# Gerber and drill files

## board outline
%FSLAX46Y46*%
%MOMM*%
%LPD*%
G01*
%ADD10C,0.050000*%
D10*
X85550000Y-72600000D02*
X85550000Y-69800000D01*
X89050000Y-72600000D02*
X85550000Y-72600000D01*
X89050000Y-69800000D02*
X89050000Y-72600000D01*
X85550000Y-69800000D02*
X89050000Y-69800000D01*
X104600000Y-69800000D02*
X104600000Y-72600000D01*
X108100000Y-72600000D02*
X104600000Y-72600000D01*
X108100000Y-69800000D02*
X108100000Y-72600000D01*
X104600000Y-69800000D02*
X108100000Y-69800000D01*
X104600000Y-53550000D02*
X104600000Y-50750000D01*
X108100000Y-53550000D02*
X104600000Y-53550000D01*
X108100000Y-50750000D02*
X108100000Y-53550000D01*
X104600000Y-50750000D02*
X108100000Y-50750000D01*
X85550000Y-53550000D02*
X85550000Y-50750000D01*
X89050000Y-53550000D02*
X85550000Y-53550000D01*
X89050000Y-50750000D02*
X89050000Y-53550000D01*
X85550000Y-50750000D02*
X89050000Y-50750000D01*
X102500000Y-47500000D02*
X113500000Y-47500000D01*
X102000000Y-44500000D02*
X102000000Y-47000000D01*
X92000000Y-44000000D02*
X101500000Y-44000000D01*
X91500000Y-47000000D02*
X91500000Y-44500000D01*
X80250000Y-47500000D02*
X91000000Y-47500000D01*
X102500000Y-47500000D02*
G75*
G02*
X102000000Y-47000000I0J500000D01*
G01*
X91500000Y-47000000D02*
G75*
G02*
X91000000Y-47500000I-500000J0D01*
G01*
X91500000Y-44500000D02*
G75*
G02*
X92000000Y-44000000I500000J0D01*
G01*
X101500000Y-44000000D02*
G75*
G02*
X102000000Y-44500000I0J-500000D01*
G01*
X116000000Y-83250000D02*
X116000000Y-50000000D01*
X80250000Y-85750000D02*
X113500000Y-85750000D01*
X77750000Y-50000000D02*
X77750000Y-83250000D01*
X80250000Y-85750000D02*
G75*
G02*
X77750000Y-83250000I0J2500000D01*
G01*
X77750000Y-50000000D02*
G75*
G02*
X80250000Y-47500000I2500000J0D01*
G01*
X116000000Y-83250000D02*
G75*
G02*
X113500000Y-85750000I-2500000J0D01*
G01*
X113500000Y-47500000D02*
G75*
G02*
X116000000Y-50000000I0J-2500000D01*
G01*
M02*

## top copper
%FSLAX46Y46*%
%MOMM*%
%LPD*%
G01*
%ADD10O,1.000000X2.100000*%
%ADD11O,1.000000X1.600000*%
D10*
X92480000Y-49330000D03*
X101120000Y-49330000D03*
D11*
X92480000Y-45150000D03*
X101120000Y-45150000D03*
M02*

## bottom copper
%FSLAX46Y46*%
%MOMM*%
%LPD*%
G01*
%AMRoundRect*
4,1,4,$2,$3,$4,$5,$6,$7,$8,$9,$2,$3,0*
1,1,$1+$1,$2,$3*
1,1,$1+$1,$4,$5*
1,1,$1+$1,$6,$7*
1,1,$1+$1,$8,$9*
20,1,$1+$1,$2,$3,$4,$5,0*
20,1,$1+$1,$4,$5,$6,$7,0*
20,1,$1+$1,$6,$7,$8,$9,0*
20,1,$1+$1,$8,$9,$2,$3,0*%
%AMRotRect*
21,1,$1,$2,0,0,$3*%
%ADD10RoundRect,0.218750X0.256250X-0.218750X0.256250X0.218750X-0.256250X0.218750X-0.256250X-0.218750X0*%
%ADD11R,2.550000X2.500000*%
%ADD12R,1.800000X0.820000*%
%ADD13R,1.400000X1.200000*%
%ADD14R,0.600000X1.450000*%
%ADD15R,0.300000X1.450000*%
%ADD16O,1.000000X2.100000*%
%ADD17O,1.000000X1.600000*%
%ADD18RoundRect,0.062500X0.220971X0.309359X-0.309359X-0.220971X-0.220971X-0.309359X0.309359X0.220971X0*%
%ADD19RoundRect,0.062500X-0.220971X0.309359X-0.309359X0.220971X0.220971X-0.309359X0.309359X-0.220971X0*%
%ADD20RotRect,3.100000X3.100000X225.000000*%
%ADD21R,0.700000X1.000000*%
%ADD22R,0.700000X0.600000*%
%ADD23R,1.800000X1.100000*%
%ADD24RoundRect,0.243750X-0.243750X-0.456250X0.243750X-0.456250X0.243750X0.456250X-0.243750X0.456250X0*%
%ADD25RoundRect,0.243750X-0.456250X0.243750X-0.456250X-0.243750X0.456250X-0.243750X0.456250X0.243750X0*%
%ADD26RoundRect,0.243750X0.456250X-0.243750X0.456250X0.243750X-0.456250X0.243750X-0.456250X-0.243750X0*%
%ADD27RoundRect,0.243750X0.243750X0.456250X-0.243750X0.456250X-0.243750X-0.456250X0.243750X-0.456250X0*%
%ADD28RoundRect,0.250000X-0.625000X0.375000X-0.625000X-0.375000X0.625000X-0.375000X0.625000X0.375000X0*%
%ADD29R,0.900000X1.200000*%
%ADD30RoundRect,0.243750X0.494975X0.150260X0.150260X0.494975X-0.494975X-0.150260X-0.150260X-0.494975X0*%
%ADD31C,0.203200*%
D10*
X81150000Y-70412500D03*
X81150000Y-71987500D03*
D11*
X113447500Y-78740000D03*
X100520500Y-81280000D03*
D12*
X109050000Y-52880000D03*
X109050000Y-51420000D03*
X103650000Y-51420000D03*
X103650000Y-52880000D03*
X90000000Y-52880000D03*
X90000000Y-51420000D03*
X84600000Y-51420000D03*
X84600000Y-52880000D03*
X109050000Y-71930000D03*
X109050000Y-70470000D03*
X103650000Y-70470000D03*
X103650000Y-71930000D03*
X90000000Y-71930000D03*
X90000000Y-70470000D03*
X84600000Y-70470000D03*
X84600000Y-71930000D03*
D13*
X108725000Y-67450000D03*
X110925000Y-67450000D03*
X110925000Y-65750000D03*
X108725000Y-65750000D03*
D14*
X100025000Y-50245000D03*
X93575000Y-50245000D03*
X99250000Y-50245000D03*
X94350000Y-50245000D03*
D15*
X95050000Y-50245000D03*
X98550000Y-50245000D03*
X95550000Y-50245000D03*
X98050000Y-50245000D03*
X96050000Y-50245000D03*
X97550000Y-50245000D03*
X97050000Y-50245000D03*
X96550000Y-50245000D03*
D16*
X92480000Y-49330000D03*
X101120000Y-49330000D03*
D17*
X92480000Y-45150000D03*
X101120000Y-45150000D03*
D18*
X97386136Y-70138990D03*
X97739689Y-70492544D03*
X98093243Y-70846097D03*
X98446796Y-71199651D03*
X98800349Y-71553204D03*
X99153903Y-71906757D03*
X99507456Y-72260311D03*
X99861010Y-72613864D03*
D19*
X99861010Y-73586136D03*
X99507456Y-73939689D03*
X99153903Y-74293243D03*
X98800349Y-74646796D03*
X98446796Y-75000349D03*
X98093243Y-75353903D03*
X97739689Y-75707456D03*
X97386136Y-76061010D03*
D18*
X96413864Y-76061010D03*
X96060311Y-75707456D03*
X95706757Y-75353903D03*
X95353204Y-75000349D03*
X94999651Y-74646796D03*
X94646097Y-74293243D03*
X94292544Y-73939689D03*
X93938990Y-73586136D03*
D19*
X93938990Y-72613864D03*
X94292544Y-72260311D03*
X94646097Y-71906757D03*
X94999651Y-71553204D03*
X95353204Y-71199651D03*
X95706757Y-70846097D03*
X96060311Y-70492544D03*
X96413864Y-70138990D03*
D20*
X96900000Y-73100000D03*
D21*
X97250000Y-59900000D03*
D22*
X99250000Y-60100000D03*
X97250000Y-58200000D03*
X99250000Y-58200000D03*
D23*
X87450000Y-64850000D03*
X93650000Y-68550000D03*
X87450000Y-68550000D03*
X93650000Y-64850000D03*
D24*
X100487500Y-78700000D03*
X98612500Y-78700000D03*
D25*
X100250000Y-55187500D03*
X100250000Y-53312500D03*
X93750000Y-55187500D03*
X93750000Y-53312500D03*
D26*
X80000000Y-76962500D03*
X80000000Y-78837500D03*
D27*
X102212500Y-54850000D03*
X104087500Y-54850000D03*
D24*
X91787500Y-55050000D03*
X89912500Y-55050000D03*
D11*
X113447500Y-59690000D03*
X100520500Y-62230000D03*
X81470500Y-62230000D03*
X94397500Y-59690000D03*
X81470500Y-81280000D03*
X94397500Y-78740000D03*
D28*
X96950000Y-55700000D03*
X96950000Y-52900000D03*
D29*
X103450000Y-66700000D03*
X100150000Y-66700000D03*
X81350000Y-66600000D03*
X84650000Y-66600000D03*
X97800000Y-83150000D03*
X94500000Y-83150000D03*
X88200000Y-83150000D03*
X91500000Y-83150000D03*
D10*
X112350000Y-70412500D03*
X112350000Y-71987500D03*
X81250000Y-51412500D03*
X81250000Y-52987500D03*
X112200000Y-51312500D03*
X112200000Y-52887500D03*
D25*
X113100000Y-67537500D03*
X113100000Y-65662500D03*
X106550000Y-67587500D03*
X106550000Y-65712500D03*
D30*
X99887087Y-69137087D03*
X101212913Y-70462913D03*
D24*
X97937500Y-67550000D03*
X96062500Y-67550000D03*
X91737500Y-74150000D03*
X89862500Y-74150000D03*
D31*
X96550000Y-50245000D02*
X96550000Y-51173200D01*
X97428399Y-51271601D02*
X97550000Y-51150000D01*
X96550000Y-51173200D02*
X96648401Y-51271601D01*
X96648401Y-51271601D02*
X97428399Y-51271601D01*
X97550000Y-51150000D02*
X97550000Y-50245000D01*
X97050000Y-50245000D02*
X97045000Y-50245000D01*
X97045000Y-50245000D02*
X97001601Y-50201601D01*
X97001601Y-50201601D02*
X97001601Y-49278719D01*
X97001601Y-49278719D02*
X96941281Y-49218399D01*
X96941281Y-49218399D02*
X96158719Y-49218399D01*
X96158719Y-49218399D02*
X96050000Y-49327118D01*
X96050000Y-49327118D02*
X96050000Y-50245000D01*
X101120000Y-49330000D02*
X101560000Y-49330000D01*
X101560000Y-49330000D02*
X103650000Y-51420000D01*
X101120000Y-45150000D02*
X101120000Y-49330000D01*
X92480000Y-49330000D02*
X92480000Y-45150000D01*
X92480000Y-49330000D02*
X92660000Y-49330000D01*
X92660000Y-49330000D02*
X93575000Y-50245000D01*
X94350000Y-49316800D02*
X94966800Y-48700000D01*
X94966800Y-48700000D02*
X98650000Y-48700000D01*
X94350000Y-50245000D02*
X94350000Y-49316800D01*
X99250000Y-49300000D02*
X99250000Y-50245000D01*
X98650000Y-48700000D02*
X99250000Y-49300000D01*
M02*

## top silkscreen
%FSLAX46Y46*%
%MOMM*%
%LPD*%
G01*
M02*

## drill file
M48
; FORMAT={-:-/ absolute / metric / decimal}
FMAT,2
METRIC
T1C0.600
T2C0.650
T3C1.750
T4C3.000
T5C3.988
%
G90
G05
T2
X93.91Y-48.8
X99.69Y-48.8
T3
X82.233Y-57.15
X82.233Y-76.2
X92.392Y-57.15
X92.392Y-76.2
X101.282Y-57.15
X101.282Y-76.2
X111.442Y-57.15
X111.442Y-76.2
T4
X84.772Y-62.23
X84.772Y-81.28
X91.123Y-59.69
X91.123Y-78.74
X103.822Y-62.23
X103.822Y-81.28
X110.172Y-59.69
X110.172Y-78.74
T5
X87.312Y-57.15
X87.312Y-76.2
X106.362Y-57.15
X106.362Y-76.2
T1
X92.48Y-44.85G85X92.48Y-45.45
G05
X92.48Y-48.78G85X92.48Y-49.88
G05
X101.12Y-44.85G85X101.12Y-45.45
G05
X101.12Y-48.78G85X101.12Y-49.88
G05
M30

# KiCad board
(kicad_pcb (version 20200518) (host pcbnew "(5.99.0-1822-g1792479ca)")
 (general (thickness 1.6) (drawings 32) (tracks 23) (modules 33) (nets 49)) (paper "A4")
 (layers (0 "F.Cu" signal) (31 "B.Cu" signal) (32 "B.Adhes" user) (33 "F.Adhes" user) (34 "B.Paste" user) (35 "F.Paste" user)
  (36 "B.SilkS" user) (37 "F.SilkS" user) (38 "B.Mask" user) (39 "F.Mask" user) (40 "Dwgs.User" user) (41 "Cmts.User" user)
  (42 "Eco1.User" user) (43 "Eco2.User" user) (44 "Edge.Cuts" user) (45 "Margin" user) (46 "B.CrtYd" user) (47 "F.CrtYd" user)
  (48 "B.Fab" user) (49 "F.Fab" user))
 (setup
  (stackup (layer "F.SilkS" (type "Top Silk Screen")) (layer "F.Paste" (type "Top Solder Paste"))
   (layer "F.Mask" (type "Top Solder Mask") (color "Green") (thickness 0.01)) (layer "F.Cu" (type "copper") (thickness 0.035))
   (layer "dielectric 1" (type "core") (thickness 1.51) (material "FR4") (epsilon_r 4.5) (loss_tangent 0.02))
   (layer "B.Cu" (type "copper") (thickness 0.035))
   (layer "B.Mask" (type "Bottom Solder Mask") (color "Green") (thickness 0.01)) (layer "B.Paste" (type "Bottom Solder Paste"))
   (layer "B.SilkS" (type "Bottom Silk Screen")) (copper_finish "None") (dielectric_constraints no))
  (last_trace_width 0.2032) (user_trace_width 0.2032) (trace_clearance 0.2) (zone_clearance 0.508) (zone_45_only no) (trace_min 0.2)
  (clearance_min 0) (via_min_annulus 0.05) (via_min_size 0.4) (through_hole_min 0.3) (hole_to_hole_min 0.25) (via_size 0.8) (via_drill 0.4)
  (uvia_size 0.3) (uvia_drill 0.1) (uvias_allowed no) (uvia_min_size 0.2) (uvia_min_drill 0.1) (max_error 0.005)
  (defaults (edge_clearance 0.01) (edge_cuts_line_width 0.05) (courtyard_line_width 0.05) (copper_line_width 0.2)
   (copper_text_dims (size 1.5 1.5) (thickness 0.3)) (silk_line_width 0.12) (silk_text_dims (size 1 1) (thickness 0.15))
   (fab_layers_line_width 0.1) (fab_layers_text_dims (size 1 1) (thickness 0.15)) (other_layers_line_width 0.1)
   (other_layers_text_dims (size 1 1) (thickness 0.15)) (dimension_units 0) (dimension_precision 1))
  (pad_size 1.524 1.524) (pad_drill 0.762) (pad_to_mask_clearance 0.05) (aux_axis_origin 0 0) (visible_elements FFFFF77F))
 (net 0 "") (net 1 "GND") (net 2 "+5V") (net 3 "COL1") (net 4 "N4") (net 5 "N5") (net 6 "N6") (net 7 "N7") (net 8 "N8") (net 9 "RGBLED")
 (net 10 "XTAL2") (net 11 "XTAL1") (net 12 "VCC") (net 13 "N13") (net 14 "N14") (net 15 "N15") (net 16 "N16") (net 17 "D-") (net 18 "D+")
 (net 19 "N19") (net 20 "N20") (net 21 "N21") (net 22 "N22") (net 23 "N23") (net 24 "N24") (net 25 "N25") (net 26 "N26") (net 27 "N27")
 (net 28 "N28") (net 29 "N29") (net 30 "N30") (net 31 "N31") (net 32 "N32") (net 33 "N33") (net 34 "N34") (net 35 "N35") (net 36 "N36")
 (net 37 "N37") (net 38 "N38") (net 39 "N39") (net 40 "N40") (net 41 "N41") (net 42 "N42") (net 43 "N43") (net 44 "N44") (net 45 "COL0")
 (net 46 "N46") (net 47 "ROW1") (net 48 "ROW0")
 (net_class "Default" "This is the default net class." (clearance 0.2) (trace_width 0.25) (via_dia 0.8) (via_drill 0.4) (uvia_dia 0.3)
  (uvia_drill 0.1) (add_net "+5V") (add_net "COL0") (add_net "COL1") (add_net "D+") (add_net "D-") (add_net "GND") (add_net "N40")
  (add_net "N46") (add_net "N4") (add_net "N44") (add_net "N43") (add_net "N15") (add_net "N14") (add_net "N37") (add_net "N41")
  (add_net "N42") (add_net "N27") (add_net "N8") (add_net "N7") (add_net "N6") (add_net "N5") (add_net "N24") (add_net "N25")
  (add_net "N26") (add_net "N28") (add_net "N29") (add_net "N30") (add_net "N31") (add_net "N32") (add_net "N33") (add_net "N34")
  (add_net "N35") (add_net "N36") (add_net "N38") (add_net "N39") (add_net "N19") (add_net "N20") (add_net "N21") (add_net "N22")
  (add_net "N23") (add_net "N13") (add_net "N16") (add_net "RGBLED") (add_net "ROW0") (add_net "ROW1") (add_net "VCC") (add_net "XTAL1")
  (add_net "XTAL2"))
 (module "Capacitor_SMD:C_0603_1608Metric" (layer "B.Cu") (at 81.15 71.2 90)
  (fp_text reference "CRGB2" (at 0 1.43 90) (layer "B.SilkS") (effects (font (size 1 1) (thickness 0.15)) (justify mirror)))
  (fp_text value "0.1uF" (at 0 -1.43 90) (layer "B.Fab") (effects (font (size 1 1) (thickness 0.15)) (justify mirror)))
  (pad "2" smd roundrect (at 0.7875 0 90) (size 0.875 0.95) (layers "B.Cu" "B.Paste" "B.Mask") (roundrect_rratio 0.25) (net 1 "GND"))
  (pad "1" smd roundrect (at -0.7875 0 90) (size 0.875 0.95) (layers "B.Cu" "B.Paste" "B.Mask") (roundrect_rratio 0.25) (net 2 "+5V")))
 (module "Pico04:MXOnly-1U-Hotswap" (layer "F.Cu") (at 106.3625 76.2 180)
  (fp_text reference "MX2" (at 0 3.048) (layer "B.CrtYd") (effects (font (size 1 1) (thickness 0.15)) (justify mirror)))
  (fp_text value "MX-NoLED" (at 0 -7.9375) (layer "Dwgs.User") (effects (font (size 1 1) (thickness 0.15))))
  (pad "" np_thru_hole circle (at 2.54 -5.08 180) (size 3 3) (drill 3) (layers *.Cu *.Mask))
  (pad "" np_thru_hole circle (at 0 0 180) (size 3.9878 3.9878) (drill 3.9878) (layers *.Cu *.Mask))
  (pad "" np_thru_hole circle (at -3.81 -2.54 180) (size 3 3) (drill 3) (layers *.Cu *.Mask))
  (pad "" np_thru_hole circle (at -5.08 0 228.0996) (size 1.75 1.75) (drill 1.75) (layers *.Cu *.Mask))
  (pad "" np_thru_hole circle (at 5.08 0 228.0996) (size 1.75 1.75) (drill 1.75) (layers *.Cu *.Mask))
  (pad "1" smd rect (at -7.085 -2.54 180) (size 2.55 2.5) (layers "B.Cu" "B.Paste" "B.Mask") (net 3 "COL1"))
  (pad "2" smd rect (at 5.842 -5.08 180) (size 2.55 2.5) (layers "B.Cu" "B.Paste" "B.Mask") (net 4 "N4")))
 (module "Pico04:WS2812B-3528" (layer "B.Cu") (at 106.35 52.15)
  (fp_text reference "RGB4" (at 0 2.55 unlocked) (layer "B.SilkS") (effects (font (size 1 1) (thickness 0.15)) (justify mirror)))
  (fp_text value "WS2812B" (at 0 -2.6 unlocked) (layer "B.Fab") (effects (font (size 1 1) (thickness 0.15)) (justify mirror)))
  (pad "1" smd rect (at 2.7 0.73) (size 1.8 0.82) (layers "B.Cu" "B.Paste" "B.Mask") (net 2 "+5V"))
  (pad "2" smd rect (at 2.7 -0.73) (size 1.8 0.82) (layers "B.Cu" "B.Paste" "B.Mask") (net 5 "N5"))
  (pad "3" smd rect (at -2.7 -0.73) (size 1.8 0.82) (layers "B.Cu" "B.Paste" "B.Mask") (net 1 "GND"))
  (pad "4" smd rect (at -2.7 0.73) (size 1.8 0.82) (layers "B.Cu" "B.Paste" "B.Mask") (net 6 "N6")))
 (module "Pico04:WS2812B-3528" (layer "B.Cu") (at 87.3 52.15)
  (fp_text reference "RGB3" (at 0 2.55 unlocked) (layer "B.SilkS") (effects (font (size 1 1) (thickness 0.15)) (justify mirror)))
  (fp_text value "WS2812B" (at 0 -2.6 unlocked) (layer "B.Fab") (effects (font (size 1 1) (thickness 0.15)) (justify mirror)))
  (pad "1" smd rect (at 2.7 0.73) (size 1.8 0.82) (layers "B.Cu" "B.Paste" "B.Mask") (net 2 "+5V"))
  (pad "2" smd rect (at 2.7 -0.73) (size 1.8 0.82) (layers "B.Cu" "B.Paste" "B.Mask") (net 6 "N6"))
  (pad "3" smd rect (at -2.7 -0.73) (size 1.8 0.82) (layers "B.Cu" "B.Paste" "B.Mask") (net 1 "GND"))
  (pad "4" smd rect (at -2.7 0.73) (size 1.8 0.82) (layers "B.Cu" "B.Paste" "B.Mask") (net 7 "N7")))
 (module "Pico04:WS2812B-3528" (layer "B.Cu") (at 106.35 71.2)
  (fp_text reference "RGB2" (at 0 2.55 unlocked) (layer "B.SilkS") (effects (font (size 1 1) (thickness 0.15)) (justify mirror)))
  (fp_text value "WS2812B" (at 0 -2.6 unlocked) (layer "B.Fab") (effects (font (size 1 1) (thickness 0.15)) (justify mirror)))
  (pad "1" smd rect (at 2.7 0.73) (size 1.8 0.82) (layers "B.Cu" "B.Paste" "B.Mask") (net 2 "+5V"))
  (pad "2" smd rect (at 2.7 -0.73) (size 1.8 0.82) (layers "B.Cu" "B.Paste" "B.Mask") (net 7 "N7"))
  (pad "3" smd rect (at -2.7 -0.73) (size 1.8 0.82) (layers "B.Cu" "B.Paste" "B.Mask") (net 1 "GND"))
  (pad "4" smd rect (at -2.7 0.73) (size 1.8 0.82) (layers "B.Cu" "B.Paste" "B.Mask") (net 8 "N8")))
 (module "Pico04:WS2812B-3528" (layer "B.Cu") (at 87.3 71.2)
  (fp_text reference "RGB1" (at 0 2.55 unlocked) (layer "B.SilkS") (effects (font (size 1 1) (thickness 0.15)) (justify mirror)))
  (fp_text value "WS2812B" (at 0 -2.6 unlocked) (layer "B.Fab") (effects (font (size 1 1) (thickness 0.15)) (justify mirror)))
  (pad "1" smd rect (at 2.7 0.73) (size 1.8 0.82) (layers "B.Cu" "B.Paste" "B.Mask") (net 2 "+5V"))
  (pad "2" smd rect (at 2.7 -0.73) (size 1.8 0.82) (layers "B.Cu" "B.Paste" "B.Mask") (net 8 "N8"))
  (pad "3" smd rect (at -2.7 -0.73) (size 1.8 0.82) (layers "B.Cu" "B.Paste" "B.Mask") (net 1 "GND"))
  (pad "4" smd rect (at -2.7 0.73) (size 1.8 0.82) (layers "B.Cu" "B.Paste" "B.Mask") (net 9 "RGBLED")))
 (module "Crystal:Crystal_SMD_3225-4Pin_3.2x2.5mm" (layer "B.Cu") (at 109.825 66.6)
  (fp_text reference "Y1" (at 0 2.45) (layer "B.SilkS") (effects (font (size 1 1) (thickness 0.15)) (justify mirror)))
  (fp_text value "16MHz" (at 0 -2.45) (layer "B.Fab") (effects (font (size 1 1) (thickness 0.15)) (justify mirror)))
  (pad "4" smd rect (at -1.1 0.85) (size 1.4 1.2) (layers "B.Cu" "B.Paste" "B.Mask") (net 1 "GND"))
  (pad "3" smd rect (at 1.1 0.85) (size 1.4 1.2) (layers "B.Cu" "B.Paste" "B.Mask") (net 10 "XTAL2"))
  (pad "2" smd rect (at 1.1 -0.85) (size 1.4 1.2) (layers "B.Cu" "B.Paste" "B.Mask") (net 1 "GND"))
  (pad "1" smd rect (at -1.1 -0.85) (size 1.4 1.2) (layers "B.Cu" "B.Paste" "B.Mask") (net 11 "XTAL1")))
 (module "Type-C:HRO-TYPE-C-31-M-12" (layer "B.Cu") (at 96.8 42.55)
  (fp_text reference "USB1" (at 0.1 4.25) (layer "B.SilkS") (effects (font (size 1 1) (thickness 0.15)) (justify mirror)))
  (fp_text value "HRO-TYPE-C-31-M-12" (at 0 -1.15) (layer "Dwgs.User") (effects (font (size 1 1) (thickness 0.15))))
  (pad "12" smd rect (at 3.225 7.695) (size 0.6 1.45) (layers "B.Cu" "B.Paste" "B.Mask") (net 1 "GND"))
  (pad "1" smd rect (at -3.225 7.695) (size 0.6 1.45) (layers "B.Cu" "B.Paste" "B.Mask") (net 1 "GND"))
  (pad "11" smd rect (at 2.45 7.695) (size 0.6 1.45) (layers "B.Cu" "B.Paste" "B.Mask") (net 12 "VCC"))
  (pad "2" smd rect (at -2.45 7.695) (size 0.6 1.45) (layers "B.Cu" "B.Paste" "B.Mask") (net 12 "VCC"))
  (pad "3" smd rect (at -1.75 7.695) (size 0.3 1.45) (layers "B.Cu" "B.Paste" "B.Mask") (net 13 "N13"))
  (pad "10" smd rect (at 1.75 7.695) (size 0.3 1.45) (layers "B.Cu" "B.Paste" "B.Mask") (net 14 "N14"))
  (pad "4" smd rect (at -1.25 7.695) (size 0.3 1.45) (layers "B.Cu" "B.Paste" "B.Mask") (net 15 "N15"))
  (pad "9" smd rect (at 1.25 7.695) (size 0.3 1.45) (layers "B.Cu" "B.Paste" "B.Mask") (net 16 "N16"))
  (pad "5" smd rect (at -0.75 7.695) (size 0.3 1.45) (layers "B.Cu" "B.Paste" "B.Mask") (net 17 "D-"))
  (pad "8" smd rect (at 0.75 7.695) (size 0.3 1.45) (layers "B.Cu" "B.Paste" "B.Mask") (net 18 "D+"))
  (pad "7" smd rect (at 0.25 7.695) (size 0.3 1.45) (layers "B.Cu" "B.Paste" "B.Mask") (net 17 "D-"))
  (pad "6" smd rect (at -0.25 7.695) (size 0.3 1.45) (layers "B.Cu" "B.Paste" "B.Mask") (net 18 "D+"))
  (pad "" np_thru_hole circle (at 2.89 6.25) (size 0.65 0.65) (drill 0.65) (layers *.Cu *.Mask))
  (pad "" np_thru_hole circle (at -2.89 6.25) (size 0.65 0.65) (drill 0.65) (layers *.Cu *.Mask))
  (pad "13" thru_hole oval (at -4.32 6.78) (size 1 2.1) (drill oval 0.6 1.7) (layers *.Cu "F.Mask") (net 1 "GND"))
  (pad "13" thru_hole oval (at 4.32 6.78) (size 1 2.1) (drill oval 0.6 1.7) (layers *.Cu "F.Mask") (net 1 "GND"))
  (pad "13" thru_hole oval (at -4.32 2.6) (size 1 1.6) (drill oval 0.6 1.2) (layers *.Cu "F.Mask") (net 1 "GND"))
  (pad "13" thru_hole oval (at 4.32 2.6) (size 1 1.6) (drill oval 0.6 1.2) (layers *.Cu "F.Mask") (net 1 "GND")))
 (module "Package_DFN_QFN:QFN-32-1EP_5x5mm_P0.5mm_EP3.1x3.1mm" (layer "B.Cu") (at 96.9 73.1 -135)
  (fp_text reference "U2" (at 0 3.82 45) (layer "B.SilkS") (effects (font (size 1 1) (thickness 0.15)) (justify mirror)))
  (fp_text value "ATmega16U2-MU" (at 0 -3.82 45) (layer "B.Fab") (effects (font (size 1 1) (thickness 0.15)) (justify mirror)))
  (pad "1" smd roundrect (at -2.4375 1.75 225) (size 0.875 0.25) (layers "B.Cu" "B.Paste" "B.Mask") (roundrect_rratio 0.25) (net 11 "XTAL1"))
  (pad "2" smd roundrect (at -2.4375 1.25 225) (size 0.875 0.25) (layers "B.Cu" "B.Paste" "B.Mask") (roundrect_rratio 0.25) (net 10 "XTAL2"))
  (pad "3" smd roundrect (at -2.4375 0.75 225) (size 0.875 0.25) (layers "B.Cu" "B.Paste" "B.Mask") (roundrect_rratio 0.25) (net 1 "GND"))
  (pad "4" smd roundrect (at -2.4375 0.25 225) (size 0.875 0.25) (layers "B.Cu" "B.Paste" "B.Mask") (roundrect_rratio 0.25) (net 2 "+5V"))
  (pad "5" smd roundrect (at -2.4375 -0.25 225) (size 0.875 0.25) (layers "B.Cu" "B.Paste" "B.Mask") (roundrect_rratio 0.25) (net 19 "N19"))
  (pad "6" smd roundrect (at -2.4375 -0.75 225) (size 0.875 0.25) (layers "B.Cu" "B.Paste" "B.Mask") (roundrect_rratio 0.25) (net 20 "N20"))
  (pad "7" smd roundrect (at -2.4375 -1.25 225) (size 0.875 0.25) (layers "B.Cu" "B.Paste" "B.Mask") (roundrect_rratio 0.25) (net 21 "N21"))
  (pad "8" smd roundrect (at -2.4375 -1.75 225) (size 0.875 0.25) (layers "B.Cu" "B.Paste" "B.Mask") (roundrect_rratio 0.25) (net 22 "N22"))
  (pad "9" smd roundrect (at -1.75 -2.4375 225) (size 0.25 0.875) (layers "B.Cu" "B.Paste" "B.Mask") (roundrect_rratio 0.25) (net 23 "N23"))
  (pad "10" smd roundrect (at -1.25 -2.4375 225) (size 0.25 0.875) (layers "B.Cu" "B.Paste" "B.Mask") (roundrect_rratio 0.25) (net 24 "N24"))
  (pad "11" smd roundrect (at -0.75 -2.4375 225) (size 0.25 0.875) (layers "B.Cu" "B.Paste" "B.Mask") (roundrect_rratio 0.25) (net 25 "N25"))
  (pad "12" smd roundrect (at -0.25 -2.4375 225) (size 0.25 0.875) (layers "B.Cu" "B.Paste" "B.Mask") (roundrect_rratio 0.25) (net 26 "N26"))
  (pad "13" smd roundrect (at 0.25 -2.4375 225) (size 0.25 0.875) (layers "B.Cu" "B.Paste" "B.Mask") (roundrect_rratio 0.25) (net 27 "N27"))
  (pad "14" smd roundrect (at 0.75 -2.4375 225) (size 0.25 0.875) (layers "B.Cu" "B.Paste" "B.Mask") (roundrect_rratio 0.25) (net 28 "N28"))
  (pad "15" smd roundrect (at 1.25 -2.4375 225) (size 0.25 0.875) (layers "B.Cu" "B.Paste" "B.Mask") (roundrect_rratio 0.25) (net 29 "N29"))
  (pad "16" smd roundrect (at 1.75 -2.4375 225) (size 0.25 0.875) (layers "B.Cu" "B.Paste" "B.Mask") (roundrect_rratio 0.25) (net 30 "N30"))
  (pad "17" smd roundrect (at 2.4375 -1.75 225) (size 0.875 0.25) (layers "B.Cu" "B.Paste" "B.Mask") (roundrect_rratio 0.25)
   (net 9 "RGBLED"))
  (pad "18" smd roundrect (at 2.4375 -1.25 225) (size 0.875 0.25) (layers "B.Cu" "B.Paste" "B.Mask") (roundrect_rratio 0.25) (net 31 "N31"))
  (pad "19" smd roundrect (at 2.4375 -0.75 225) (size 0.875 0.25) (layers "B.Cu" "B.Paste" "B.Mask") (roundrect_rratio 0.25) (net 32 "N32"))
  (pad "20" smd roundrect (at 2.4375 -0.25 225) (size 0.875 0.25) (layers "B.Cu" "B.Paste" "B.Mask") (roundrect_rratio 0.25) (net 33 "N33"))
  (pad "21" smd roundrect (at 2.4375 0.25 225) (size 0.875 0.25) (layers "B.Cu" "B.Paste" "B.Mask") (roundrect_rratio 0.25) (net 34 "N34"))
  (pad "22" smd roundrect (at 2.4375 0.75 225) (size 0.875 0.25) (layers "B.Cu" "B.Paste" "B.Mask") (roundrect_rratio 0.25) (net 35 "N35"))
  (pad "23" smd roundrect (at 2.4375 1.25 225) (size 0.875 0.25) (layers "B.Cu" "B.Paste" "B.Mask") (roundrect_rratio 0.25) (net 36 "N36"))
  (pad "24" smd roundrect (at 2.4375 1.75 225) (size 0.875 0.25) (layers "B.Cu" "B.Paste" "B.Mask") (roundrect_rratio 0.25) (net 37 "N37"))
  (pad "25" smd roundrect (at 1.75 2.4375 225) (size 0.25 0.875) (layers "B.Cu" "B.Paste" "B.Mask") (roundrect_rratio 0.25) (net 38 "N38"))
  (pad "26" smd roundrect (at 1.25 2.4375 225) (size 0.25 0.875) (layers "B.Cu" "B.Paste" "B.Mask") (roundrect_rratio 0.25) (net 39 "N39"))
  (pad "27" smd roundrect (at 0.75 2.4375 225) (size 0.25 0.875) (layers "B.Cu" "B.Paste" "B.Mask") (roundrect_rratio 0.25) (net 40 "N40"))
  (pad "28" smd roundrect (at 0.25 2.4375 225) (size 0.25 0.875) (layers "B.Cu" "B.Paste" "B.Mask") (roundrect_rratio 0.25) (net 1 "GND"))
  (pad "29" smd roundrect (at -0.25 2.4375 225) (size 0.25 0.875) (layers "B.Cu" "B.Paste" "B.Mask") (roundrect_rratio 0.25) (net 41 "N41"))
  (pad "30" smd roundrect (at -0.75 2.4375 225) (size 0.25 0.875) (layers "B.Cu" "B.Paste" "B.Mask") (roundrect_rratio 0.25) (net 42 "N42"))
  (pad "31" smd roundrect (at -1.25 2.4375 225) (size 0.25 0.875) (layers "B.Cu" "B.Paste" "B.Mask") (roundrect_rratio 0.25) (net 2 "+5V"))
  (pad "32" smd roundrect (at -1.75 2.4375 225) (size 0.25 0.875) (layers "B.Cu" "B.Paste" "B.Mask") (roundrect_rratio 0.25) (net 2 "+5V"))
  (pad "33" smd rect (at 0 0 225) (size 3.1 3.1) (layers "B.Cu" "B.Mask") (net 1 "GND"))
  (pad "" smd roundrect (at -1.03 1.03 225) (size 0.83 0.83) (layers "B.Paste") (roundrect_rratio 0.25))
  (pad "" smd roundrect (at -1.03 0 225) (size 0.83 0.83) (layers "B.Paste") (roundrect_rratio 0.25))
  (pad "" smd roundrect (at -1.03 -1.03 225) (size 0.83 0.83) (layers "B.Paste") (roundrect_rratio 0.25))
  (pad "" smd roundrect (at 0 1.03 225) (size 0.83 0.83) (layers "B.Paste") (roundrect_rratio 0.25))
  (pad "" smd roundrect (at 0 0 225) (size 0.83 0.83) (layers "B.Paste") (roundrect_rratio 0.25))
  (pad "" smd roundrect (at 0 -1.03 225) (size 0.83 0.83) (layers "B.Paste") (roundrect_rratio 0.25))
  (pad "" smd roundrect (at 1.03 1.03 225) (size 0.83 0.83) (layers "B.Paste") (roundrect_rratio 0.25))
  (pad "" smd roundrect (at 1.03 0 225) (size 0.83 0.83) (layers "B.Paste") (roundrect_rratio 0.25))
  (pad "" smd roundrect (at 1.03 -1.03 225) (size 0.83 0.83) (layers "B.Paste") (roundrect_rratio 0.25)))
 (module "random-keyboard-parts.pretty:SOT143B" (layer "B.Cu") (at 98.25 59.15)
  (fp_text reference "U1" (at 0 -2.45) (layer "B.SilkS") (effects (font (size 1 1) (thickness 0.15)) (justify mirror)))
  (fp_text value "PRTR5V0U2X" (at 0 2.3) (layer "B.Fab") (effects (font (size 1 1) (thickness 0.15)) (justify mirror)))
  (pad "1" smd rect (at -1 0.75 90) (size 1 0.7) (layers "B.Cu" "B.Paste" "B.Mask") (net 1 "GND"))
  (pad "4" smd rect (at 1 0.95 90) (size 0.6 0.7) (layers "B.Cu" "B.Paste" "B.Mask") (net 12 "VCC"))
  (pad "2" smd rect (at -1 -0.95 90) (size 0.6 0.7) (layers "B.Cu" "B.Paste" "B.Mask") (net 18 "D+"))
  (pad "3" smd rect (at 1 -0.95 90) (size 0.6 0.7) (layers "B.Cu" "B.Paste" "B.Mask") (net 17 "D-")))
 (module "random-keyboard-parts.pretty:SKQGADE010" (layer "B.Cu") (at 90.55 66.7)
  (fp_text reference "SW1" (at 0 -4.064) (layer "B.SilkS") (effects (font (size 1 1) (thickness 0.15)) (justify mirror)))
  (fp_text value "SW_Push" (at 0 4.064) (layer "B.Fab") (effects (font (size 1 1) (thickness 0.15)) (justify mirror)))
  (pad "4" smd rect (at -3.1 -1.85) (size 1.8 1.1) (layers "B.Cu" "B.Paste" "B.Mask"))
  (pad "3" smd rect (at 3.1 1.85) (size 1.8 1.1) (layers "B.Cu" "B.Paste" "B.Mask"))
  (pad "2" smd rect (at -3.1 1.85) (size 1.8 1.1) (layers "B.Cu" "B.Paste" "B.Mask") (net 37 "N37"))
  (pad "1" smd rect (at 3.1 -1.85) (size 1.8 1.1) (layers "B.Cu" "B.Paste" "B.Mask") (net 1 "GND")))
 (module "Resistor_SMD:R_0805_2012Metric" (layer "B.Cu") (at 99.55 78.7)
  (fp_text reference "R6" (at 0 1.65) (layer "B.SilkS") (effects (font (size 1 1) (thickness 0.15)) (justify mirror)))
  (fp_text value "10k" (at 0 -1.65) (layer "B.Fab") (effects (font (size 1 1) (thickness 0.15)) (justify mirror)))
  (pad "2" smd roundrect (at 0.9375 0) (size 0.975 1.4) (layers "B.Cu" "B.Paste" "B.Mask") (roundrect_rratio 0.25) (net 1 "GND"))
  (pad "1" smd roundrect (at -0.9375 0) (size 0.975 1.4) (layers "B.Cu" "B.Paste" "B.Mask") (roundrect_rratio 0.25) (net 27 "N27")))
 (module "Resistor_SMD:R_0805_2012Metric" (layer "B.Cu") (at 100.25 54.25 -90)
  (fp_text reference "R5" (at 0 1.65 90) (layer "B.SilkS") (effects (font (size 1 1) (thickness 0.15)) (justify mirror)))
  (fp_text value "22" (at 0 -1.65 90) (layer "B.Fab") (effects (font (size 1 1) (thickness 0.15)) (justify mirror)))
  (pad "2" smd roundrect (at 0.9375 0 270) (size 0.975 1.4) (layers "B.Cu" "B.Paste" "B.Mask") (roundrect_rratio 0.25) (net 42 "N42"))
  (pad "1" smd roundrect (at -0.9375 0 270) (size 0.975 1.4) (layers "B.Cu" "B.Paste" "B.Mask") (roundrect_rratio 0.25) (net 17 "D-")))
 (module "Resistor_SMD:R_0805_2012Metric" (layer "B.Cu") (at 93.75 54.25 -90)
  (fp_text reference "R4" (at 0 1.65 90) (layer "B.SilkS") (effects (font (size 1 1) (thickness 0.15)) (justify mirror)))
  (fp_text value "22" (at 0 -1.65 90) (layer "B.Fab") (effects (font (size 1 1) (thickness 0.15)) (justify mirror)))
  (pad "2" smd roundrect (at 0.9375 0 270) (size 0.975 1.4) (layers "B.Cu" "B.Paste" "B.Mask") (roundrect_rratio 0.25) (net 41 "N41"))
  (pad "1" smd roundrect (at -0.9375 0 270) (size 0.975 1.4) (layers "B.Cu" "B.Paste" "B.Mask") (roundrect_rratio 0.25) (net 18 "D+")))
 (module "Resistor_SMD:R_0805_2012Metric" (layer "B.Cu") (at 80 77.9 90)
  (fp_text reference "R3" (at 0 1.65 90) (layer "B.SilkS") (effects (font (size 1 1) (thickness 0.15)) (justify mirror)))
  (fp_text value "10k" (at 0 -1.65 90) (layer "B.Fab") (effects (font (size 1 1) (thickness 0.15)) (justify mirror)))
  (pad "2" smd roundrect (at 0.9375 0 90) (size 0.975 1.4) (layers "B.Cu" "B.Paste" "B.Mask") (roundrect_rratio 0.25) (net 37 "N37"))
  (pad "1" smd roundrect (at -0.9375 0 90) (size 0.975 1.4) (layers "B.Cu" "B.Paste" "B.Mask") (roundrect_rratio 0.25) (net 2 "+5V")))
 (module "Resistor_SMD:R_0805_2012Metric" (layer "B.Cu") (at 103.15 54.85 180)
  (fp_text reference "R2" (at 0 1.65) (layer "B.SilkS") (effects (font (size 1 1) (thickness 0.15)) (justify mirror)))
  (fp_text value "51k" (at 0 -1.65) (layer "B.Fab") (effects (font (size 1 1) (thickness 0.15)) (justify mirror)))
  (pad "2" smd roundrect (at 0.9375 0 180) (size 0.975 1.4) (layers "B.Cu" "B.Paste" "B.Mask") (roundrect_rratio 0.25) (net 14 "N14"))
  (pad "1" smd roundrect (at -0.9375 0 180) (size 0.975 1.4) (layers "B.Cu" "B.Paste" "B.Mask") (roundrect_rratio 0.25) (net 1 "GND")))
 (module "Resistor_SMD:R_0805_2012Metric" (layer "B.Cu") (at 90.85 55.05)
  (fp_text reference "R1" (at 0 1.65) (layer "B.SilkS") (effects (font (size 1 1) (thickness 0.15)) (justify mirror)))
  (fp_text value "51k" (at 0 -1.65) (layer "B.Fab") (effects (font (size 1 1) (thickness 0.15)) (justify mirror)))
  (pad "2" smd roundrect (at 0.9375 0) (size 0.975 1.4) (layers "B.Cu" "B.Paste" "B.Mask") (roundrect_rratio 0.25) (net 15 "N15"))
  (pad "1" smd roundrect (at -0.9375 0) (size 0.975 1.4) (layers "B.Cu" "B.Paste" "B.Mask") (roundrect_rratio 0.25) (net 1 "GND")))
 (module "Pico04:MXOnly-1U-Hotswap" (layer "F.Cu") (at 106.3625 57.15 180)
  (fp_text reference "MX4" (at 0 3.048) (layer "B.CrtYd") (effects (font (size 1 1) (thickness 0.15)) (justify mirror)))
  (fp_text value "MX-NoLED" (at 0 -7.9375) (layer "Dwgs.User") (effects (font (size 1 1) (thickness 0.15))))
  (pad "" np_thru_hole circle (at 2.54 -5.08 180) (size 3 3) (drill 3) (layers *.Cu *.Mask))
  (pad "" np_thru_hole circle (at 0 0 180) (size 3.9878 3.9878) (drill 3.9878) (layers *.Cu *.Mask))
  (pad "" np_thru_hole circle (at -3.81 -2.54 180) (size 3 3) (drill 3) (layers *.Cu *.Mask))
  (pad "" np_thru_hole circle (at -5.08 0 228.0996) (size 1.75 1.75) (drill 1.75) (layers *.Cu *.Mask))
  (pad "" np_thru_hole circle (at 5.08 0 228.0996) (size 1.75 1.75) (drill 1.75) (layers *.Cu *.Mask))
  (pad "1" smd rect (at -7.085 -2.54 180) (size 2.55 2.5) (layers "B.Cu" "B.Paste" "B.Mask") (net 3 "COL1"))
  (pad "2" smd rect (at 5.842 -5.08 180) (size 2.55 2.5) (layers "B.Cu" "B.Paste" "B.Mask") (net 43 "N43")))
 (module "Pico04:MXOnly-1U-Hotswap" (layer "F.Cu") (at 87.3125 57.15 180)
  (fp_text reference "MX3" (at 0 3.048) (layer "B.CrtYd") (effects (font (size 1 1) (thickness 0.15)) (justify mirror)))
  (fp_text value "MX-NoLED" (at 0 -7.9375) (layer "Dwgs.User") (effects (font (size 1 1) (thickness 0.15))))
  (pad "2" smd rect (at 5.842 -5.08 180) (size 2.55 2.5) (layers "B.Cu" "B.Paste" "B.Mask") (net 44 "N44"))
  (pad "1" smd rect (at -7.085 -2.54 180) (size 2.55 2.5) (layers "B.Cu" "B.Paste" "B.Mask") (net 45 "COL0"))
  (pad "" np_thru_hole circle (at 5.08 0 228.0996) (size 1.75 1.75) (drill 1.75) (layers *.Cu *.Mask))
  (pad "" np_thru_hole circle (at -5.08 0 228.0996) (size 1.75 1.75) (drill 1.75) (layers *.Cu *.Mask))
  (pad "" np_thru_hole circle (at -3.81 -2.54 180) (size 3 3) (drill 3) (layers *.Cu *.Mask))
  (pad "" np_thru_hole circle (at 0 0 180) (size 3.9878 3.9878) (drill 3.9878) (layers *.Cu *.Mask))
  (pad "" np_thru_hole circle (at 2.54 -5.08 180) (size 3 3) (drill 3) (layers *.Cu *.Mask)))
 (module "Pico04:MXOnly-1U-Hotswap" (layer "F.Cu") (at 87.3125 76.2 180)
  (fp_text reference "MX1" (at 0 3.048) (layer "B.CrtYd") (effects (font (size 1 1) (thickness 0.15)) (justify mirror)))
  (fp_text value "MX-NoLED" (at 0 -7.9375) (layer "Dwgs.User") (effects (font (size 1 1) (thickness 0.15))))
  (pad "2" smd rect (at 5.842 -5.08 180) (size 2.55 2.5) (layers "B.Cu" "B.Paste" "B.Mask") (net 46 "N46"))
  (pad "1" smd rect (at -7.085 -2.54 180) (size 2.55 2.5) (layers "B.Cu" "B.Paste" "B.Mask") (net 45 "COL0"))
  (pad "" np_thru_hole circle (at 5.08 0 228.0996) (size 1.75 1.75) (drill 1.75) (layers *.Cu *.Mask))
  (pad "" np_thru_hole circle (at -5.08 0 228.0996) (size 1.75 1.75) (drill 1.75) (layers *.Cu *.Mask))
  (pad "" np_thru_hole circle (at -3.81 -2.54 180) (size 3 3) (drill 3) (layers *.Cu *.Mask))
  (pad "" np_thru_hole circle (at 0 0 180) (size 3.9878 3.9878) (drill 3.9878) (layers *.Cu *.Mask))
  (pad "" np_thru_hole circle (at 2.54 -5.08 180) (size 3 3) (drill 3) (layers *.Cu *.Mask)))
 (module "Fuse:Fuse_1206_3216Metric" (layer "B.Cu") (at 96.95 54.3 -90)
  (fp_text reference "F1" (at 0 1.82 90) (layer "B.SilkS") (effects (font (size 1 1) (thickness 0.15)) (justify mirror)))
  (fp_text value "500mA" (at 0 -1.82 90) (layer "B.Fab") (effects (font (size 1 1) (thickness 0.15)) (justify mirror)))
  (pad "2" smd roundrect (at 1.4 0 270) (size 1.25 1.75) (layers "B.Cu" "B.Paste" "B.Mask") (roundrect_rratio 0.2) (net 2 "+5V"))
  (pad "1" smd roundrect (at -1.4 0 270) (size 1.25 1.75) (layers "B.Cu" "B.Paste" "B.Mask") (roundrect_rratio 0.2) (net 12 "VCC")))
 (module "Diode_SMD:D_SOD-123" (layer "B.Cu") (at 101.8 66.7)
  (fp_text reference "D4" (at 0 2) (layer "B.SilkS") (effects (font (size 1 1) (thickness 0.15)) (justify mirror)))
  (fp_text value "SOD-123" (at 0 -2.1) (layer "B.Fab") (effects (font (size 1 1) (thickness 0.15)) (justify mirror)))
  (pad "2" smd rect (at 1.65 0) (size 0.9 1.2) (layers "B.Cu" "B.Paste" "B.Mask") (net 43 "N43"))
  (pad "1" smd rect (at -1.65 0) (size 0.9 1.2) (layers "B.Cu" "B.Paste" "B.Mask") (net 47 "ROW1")))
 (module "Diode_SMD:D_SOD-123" (layer "B.Cu") (at 83 66.6 180)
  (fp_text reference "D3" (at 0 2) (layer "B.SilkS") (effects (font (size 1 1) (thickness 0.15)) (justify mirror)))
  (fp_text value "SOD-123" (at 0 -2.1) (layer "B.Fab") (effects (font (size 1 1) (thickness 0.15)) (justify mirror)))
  (pad "2" smd rect (at 1.65 0 180) (size 0.9 1.2) (layers "B.Cu" "B.Paste" "B.Mask") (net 44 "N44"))
  (pad "1" smd rect (at -1.65 0 180) (size 0.9 1.2) (layers "B.Cu" "B.Paste" "B.Mask") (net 47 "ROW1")))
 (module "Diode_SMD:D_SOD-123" (layer "B.Cu") (at 96.15 83.15)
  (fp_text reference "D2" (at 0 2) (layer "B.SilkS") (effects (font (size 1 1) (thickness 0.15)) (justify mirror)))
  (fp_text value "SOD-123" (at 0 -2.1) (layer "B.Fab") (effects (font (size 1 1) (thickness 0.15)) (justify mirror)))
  (pad "2" smd rect (at 1.65 0) (size 0.9 1.2) (layers "B.Cu" "B.Paste" "B.Mask") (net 4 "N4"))
  (pad "1" smd rect (at -1.65 0) (size 0.9 1.2) (layers "B.Cu" "B.Paste" "B.Mask") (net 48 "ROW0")))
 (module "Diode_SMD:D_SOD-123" (layer "B.Cu") (at 89.85 83.15 180)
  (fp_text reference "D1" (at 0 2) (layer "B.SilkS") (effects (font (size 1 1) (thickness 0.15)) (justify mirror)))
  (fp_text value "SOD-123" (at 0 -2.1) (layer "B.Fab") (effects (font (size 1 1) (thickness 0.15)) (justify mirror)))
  (pad "2" smd rect (at 1.65 0 180) (size 0.9 1.2) (layers "B.Cu" "B.Paste" "B.Mask") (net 46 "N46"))
  (pad "1" smd rect (at -1.65 0 180) (size 0.9 1.2) (layers "B.Cu" "B.Paste" "B.Mask") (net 48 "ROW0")))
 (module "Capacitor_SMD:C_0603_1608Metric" (layer "B.Cu") (at 112.35 71.2 90)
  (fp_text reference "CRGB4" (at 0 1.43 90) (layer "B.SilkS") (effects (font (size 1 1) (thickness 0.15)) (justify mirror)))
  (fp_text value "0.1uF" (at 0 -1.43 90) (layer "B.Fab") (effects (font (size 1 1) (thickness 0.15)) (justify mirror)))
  (pad "2" smd roundrect (at 0.7875 0 90) (size 0.875 0.95) (layers "B.Cu" "B.Paste" "B.Mask") (roundrect_rratio 0.25) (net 1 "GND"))
  (pad "1" smd roundrect (at -0.7875 0 90) (size 0.875 0.95) (layers "B.Cu" "B.Paste" "B.Mask") (roundrect_rratio 0.25) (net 2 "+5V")))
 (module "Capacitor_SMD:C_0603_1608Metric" (layer "B.Cu") (at 81.25 52.2 90)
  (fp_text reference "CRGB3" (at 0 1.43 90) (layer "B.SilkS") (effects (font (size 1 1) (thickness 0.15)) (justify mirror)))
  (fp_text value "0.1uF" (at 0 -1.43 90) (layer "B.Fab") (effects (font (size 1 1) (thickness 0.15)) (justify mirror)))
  (pad "2" smd roundrect (at 0.7875 0 90) (size 0.875 0.95) (layers "B.Cu" "B.Paste" "B.Mask") (roundrect_rratio 0.25) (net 1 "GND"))
  (pad "1" smd roundrect (at -0.7875 0 90) (size 0.875 0.95) (layers "B.Cu" "B.Paste" "B.Mask") (roundrect_rratio 0.25) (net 2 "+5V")))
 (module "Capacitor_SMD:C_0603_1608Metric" (layer "B.Cu") (at 112.2 52.1 90)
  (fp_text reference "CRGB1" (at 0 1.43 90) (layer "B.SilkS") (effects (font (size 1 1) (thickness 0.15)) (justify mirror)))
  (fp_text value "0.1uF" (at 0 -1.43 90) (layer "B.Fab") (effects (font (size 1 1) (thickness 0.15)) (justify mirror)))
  (pad "2" smd roundrect (at 0.7875 0 90) (size 0.875 0.95) (layers "B.Cu" "B.Paste" "B.Mask") (roundrect_rratio 0.25) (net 1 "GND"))
  (pad "1" smd roundrect (at -0.7875 0 90) (size 0.875 0.95) (layers "B.Cu" "B.Paste" "B.Mask") (roundrect_rratio 0.25) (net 2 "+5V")))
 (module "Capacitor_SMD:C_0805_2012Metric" (layer "B.Cu") (at 113.1 66.6 -90)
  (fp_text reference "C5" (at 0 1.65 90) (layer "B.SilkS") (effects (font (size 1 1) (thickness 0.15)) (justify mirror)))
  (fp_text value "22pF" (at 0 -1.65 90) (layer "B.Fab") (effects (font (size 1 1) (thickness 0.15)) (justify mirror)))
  (pad "2" smd roundrect (at 0.9375 0 270) (size 0.975 1.4) (layers "B.Cu" "B.Paste" "B.Mask") (roundrect_rratio 0.25) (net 10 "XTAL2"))
  (pad "1" smd roundrect (at -0.9375 0 270) (size 0.975 1.4) (layers "B.Cu" "B.Paste" "B.Mask") (roundrect_rratio 0.25) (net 1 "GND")))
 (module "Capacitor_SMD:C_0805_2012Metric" (layer "B.Cu") (at 106.55 66.65 -90)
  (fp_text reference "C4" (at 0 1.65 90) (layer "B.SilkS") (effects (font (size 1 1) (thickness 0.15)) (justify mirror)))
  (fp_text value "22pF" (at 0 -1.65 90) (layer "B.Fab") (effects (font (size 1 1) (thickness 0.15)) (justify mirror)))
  (pad "2" smd roundrect (at 0.9375 0 270) (size 0.975 1.4) (layers "B.Cu" "B.Paste" "B.Mask") (roundrect_rratio 0.25) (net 1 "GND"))
  (pad "1" smd roundrect (at -0.9375 0 270) (size 0.975 1.4) (layers "B.Cu" "B.Paste" "B.Mask") (roundrect_rratio 0.25) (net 11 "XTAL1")))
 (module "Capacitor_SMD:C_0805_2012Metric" (layer "B.Cu") (at 100.55 69.8 135)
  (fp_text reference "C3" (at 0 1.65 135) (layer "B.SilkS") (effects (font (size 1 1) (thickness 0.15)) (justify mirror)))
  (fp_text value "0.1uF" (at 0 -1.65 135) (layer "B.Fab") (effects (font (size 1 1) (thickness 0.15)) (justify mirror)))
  (pad "2" smd roundrect (at 0.9375 0 135) (size 0.975 1.4) (layers "B.Cu" "B.Paste" "B.Mask") (roundrect_rratio 0.25) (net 1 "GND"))
  (pad "1" smd roundrect (at -0.9375 0 135) (size 0.975 1.4) (layers "B.Cu" "B.Paste" "B.Mask") (roundrect_rratio 0.25) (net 2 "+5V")))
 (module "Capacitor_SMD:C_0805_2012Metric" (layer "B.Cu") (at 97 67.55)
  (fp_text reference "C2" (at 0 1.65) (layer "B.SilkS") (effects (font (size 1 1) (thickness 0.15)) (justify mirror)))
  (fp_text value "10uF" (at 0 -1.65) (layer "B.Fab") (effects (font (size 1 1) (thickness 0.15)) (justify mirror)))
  (pad "2" smd roundrect (at 0.9375 0) (size 0.975 1.4) (layers "B.Cu" "B.Paste" "B.Mask") (roundrect_rratio 0.25) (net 1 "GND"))
  (pad "1" smd roundrect (at -0.9375 0) (size 0.975 1.4) (layers "B.Cu" "B.Paste" "B.Mask") (roundrect_rratio 0.25) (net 2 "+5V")))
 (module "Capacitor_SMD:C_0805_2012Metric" (layer "B.Cu") (at 90.8 74.15)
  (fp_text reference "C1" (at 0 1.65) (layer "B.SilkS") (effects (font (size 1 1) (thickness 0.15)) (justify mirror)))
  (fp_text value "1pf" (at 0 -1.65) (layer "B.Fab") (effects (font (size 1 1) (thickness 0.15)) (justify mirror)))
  (pad "2" smd roundrect (at 0.9375 0) (size 0.975 1.4) (layers "B.Cu" "B.Paste" "B.Mask") (roundrect_rratio 0.25) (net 1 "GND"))
  (pad "1" smd roundrect (at -0.9375 0) (size 0.975 1.4) (layers "B.Cu" "B.Paste" "B.Mask") (roundrect_rratio 0.25) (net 40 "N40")))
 (gr_line (start 85.55 72.6) (end 85.55 69.8) (layer "Edge.Cuts") (width 0.05))
 (gr_line (start 89.05 72.6) (end 85.55 72.6) (layer "Edge.Cuts") (width 0.05))
 (gr_line (start 89.05 69.8) (end 89.05 72.6) (layer "Edge.Cuts") (width 0.05))
 (gr_line (start 85.55 69.8) (end 89.05 69.8) (layer "Edge.Cuts") (width 0.05))
 (gr_line (start 104.6 69.8) (end 104.6 72.6) (layer "Edge.Cuts") (width 0.05))
 (gr_line (start 108.1 72.6) (end 104.6 72.6) (layer "Edge.Cuts") (width 0.05))
 (gr_line (start 108.1 69.8) (end 108.1 72.6) (layer "Edge.Cuts") (width 0.05))
 (gr_line (start 104.6 69.8) (end 108.1 69.8) (layer "Edge.Cuts") (width 0.05))
 (gr_line (start 104.6 53.55) (end 104.6 50.75) (layer "Edge.Cuts") (width 0.05))
 (gr_line (start 108.1 53.55) (end 104.6 53.55) (layer "Edge.Cuts") (width 0.05))
 (gr_line (start 108.1 50.75) (end 108.1 53.55) (layer "Edge.Cuts") (width 0.05))
 (gr_line (start 104.6 50.75) (end 108.1 50.75) (layer "Edge.Cuts") (width 0.05))
 (gr_line (start 85.55 53.55) (end 85.55 50.75) (layer "Edge.Cuts") (width 0.05))
 (gr_line (start 89.05 53.55) (end 85.55 53.55) (layer "Edge.Cuts") (width 0.05))
 (gr_line (start 89.05 50.75) (end 89.05 53.55) (layer "Edge.Cuts") (width 0.05))
 (gr_line (start 85.55 50.75) (end 89.05 50.75) (layer "Edge.Cuts") (width 0.05))
 (gr_line (start 102.5 47.5) (end 113.5 47.5) (layer "Edge.Cuts") (width 0.05))
 (gr_line (start 102 44.5) (end 102 47) (layer "Edge.Cuts") (width 0.05))
 (gr_line (start 92 44) (end 101.5 44) (layer "Edge.Cuts") (width 0.05))
 (gr_line (start 91.5 47) (end 91.5 44.5) (layer "Edge.Cuts") (width 0.05))
 (gr_line (start 80.25 47.5) (end 91 47.5) (layer "Edge.Cuts") (width 0.05))
 (gr_arc (start 102.5 47) (end 102 47) (angle -90) (layer "Edge.Cuts") (width 0.05))
 (gr_arc (start 91 47) (end 91 47.5) (angle -90) (layer "Edge.Cuts") (width 0.05))
 (gr_arc (start 92 44.5) (end 92 44) (angle -90) (layer "Edge.Cuts") (width 0.05))
 (gr_arc (start 101.5 44.5) (end 102 44.5) (angle -90) (layer "Edge.Cuts") (width 0.05))
 (gr_line (start 116 83.25) (end 116 50) (layer "Edge.Cuts") (width 0.05))
 (gr_line (start 80.25 85.75) (end 113.5 85.75) (layer "Edge.Cuts") (width 0.05))
 (gr_line (start 77.75 50) (end 77.75 83.25) (layer "Edge.Cuts") (width 0.05))
 (gr_arc (start 80.25 83.25) (end 77.75 83.25) (angle -90) (layer "Edge.Cuts") (width 0.05))
 (gr_arc (start 80.25 50) (end 80.25 47.5) (angle -90) (layer "Edge.Cuts") (width 0.05))
 (gr_arc (start 113.5 83.25) (end 113.5 85.75) (angle -90) (layer "Edge.Cuts") (width 0.05))
 (gr_arc (start 113.5 50) (end 116 50) (angle -90) (layer "Edge.Cuts") (width 0.05))
 (segment (start 96.55 50.245) (end 96.55 51.1732) (width 0.2032) (layer "B.Cu") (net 18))
 (segment (start 97.428399 51.271601) (end 97.55 51.15) (width 0.2032) (layer "B.Cu") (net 18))
 (segment (start 96.55 51.1732) (end 96.648401 51.271601) (width 0.2032) (layer "B.Cu") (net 18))
 (segment (start 96.648401 51.271601) (end 97.428399 51.271601) (width 0.2032) (layer "B.Cu") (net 18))
 (segment (start 97.55 51.15) (end 97.55 50.245) (width 0.2032) (layer "B.Cu") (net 18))
 (segment (start 97.05 50.245) (end 97.045 50.245) (width 0.2032) (layer "B.Cu") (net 17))
 (segment (start 97.045 50.245) (end 97.001601 50.201601) (width 0.2032) (layer "B.Cu") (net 17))
 (segment (start 97.001601 50.201601) (end 97.001601 49.278719) (width 0.2032) (layer "B.Cu") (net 17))
 (segment (start 97.001601 49.278719) (end 96.941281 49.218399) (width 0.2032) (layer "B.Cu") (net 17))
 (segment (start 96.941281 49.218399) (end 96.158719 49.218399) (width 0.2032) (layer "B.Cu") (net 17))
 (segment (start 96.158719 49.218399) (end 96.05 49.327118) (width 0.2032) (layer "B.Cu") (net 17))
 (segment (start 96.05 49.327118) (end 96.05 50.245) (width 0.2032) (layer "B.Cu") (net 17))
 (segment (start 101.12 49.33) (end 101.56 49.33) (width 0.2032) (layer "B.Cu") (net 1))
 (segment (start 101.56 49.33) (end 103.65 51.42) (width 0.2032) (layer "B.Cu") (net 1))
 (segment (start 101.12 45.15) (end 101.12 49.33) (width 0.2032) (layer "B.Cu") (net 1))
 (segment (start 92.48 49.33) (end 92.48 45.15) (width 0.2032) (layer "B.Cu") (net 1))
 (segment (start 92.48 49.33) (end 92.66 49.33) (width 0.2032) (layer "B.Cu") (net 1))
 (segment (start 92.66 49.33) (end 93.575 50.245) (width 0.2032) (layer "B.Cu") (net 1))
 (segment (start 94.35 49.3168) (end 94.9668 48.7) (width 0.2032) (layer "B.Cu") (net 12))
 (segment (start 94.9668 48.7) (end 98.65 48.7) (width 0.2032) (layer "B.Cu") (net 12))
 (segment (start 94.35 50.245) (end 94.35 49.3168) (width 0.2032) (layer "B.Cu") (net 12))
 (segment (start 99.25 49.3) (end 99.25 50.245) (width 0.2032) (layer "B.Cu") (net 12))
 (segment (start 98.65 48.7) (end 99.25 49.3) (width 0.2032) (layer "B.Cu") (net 12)))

